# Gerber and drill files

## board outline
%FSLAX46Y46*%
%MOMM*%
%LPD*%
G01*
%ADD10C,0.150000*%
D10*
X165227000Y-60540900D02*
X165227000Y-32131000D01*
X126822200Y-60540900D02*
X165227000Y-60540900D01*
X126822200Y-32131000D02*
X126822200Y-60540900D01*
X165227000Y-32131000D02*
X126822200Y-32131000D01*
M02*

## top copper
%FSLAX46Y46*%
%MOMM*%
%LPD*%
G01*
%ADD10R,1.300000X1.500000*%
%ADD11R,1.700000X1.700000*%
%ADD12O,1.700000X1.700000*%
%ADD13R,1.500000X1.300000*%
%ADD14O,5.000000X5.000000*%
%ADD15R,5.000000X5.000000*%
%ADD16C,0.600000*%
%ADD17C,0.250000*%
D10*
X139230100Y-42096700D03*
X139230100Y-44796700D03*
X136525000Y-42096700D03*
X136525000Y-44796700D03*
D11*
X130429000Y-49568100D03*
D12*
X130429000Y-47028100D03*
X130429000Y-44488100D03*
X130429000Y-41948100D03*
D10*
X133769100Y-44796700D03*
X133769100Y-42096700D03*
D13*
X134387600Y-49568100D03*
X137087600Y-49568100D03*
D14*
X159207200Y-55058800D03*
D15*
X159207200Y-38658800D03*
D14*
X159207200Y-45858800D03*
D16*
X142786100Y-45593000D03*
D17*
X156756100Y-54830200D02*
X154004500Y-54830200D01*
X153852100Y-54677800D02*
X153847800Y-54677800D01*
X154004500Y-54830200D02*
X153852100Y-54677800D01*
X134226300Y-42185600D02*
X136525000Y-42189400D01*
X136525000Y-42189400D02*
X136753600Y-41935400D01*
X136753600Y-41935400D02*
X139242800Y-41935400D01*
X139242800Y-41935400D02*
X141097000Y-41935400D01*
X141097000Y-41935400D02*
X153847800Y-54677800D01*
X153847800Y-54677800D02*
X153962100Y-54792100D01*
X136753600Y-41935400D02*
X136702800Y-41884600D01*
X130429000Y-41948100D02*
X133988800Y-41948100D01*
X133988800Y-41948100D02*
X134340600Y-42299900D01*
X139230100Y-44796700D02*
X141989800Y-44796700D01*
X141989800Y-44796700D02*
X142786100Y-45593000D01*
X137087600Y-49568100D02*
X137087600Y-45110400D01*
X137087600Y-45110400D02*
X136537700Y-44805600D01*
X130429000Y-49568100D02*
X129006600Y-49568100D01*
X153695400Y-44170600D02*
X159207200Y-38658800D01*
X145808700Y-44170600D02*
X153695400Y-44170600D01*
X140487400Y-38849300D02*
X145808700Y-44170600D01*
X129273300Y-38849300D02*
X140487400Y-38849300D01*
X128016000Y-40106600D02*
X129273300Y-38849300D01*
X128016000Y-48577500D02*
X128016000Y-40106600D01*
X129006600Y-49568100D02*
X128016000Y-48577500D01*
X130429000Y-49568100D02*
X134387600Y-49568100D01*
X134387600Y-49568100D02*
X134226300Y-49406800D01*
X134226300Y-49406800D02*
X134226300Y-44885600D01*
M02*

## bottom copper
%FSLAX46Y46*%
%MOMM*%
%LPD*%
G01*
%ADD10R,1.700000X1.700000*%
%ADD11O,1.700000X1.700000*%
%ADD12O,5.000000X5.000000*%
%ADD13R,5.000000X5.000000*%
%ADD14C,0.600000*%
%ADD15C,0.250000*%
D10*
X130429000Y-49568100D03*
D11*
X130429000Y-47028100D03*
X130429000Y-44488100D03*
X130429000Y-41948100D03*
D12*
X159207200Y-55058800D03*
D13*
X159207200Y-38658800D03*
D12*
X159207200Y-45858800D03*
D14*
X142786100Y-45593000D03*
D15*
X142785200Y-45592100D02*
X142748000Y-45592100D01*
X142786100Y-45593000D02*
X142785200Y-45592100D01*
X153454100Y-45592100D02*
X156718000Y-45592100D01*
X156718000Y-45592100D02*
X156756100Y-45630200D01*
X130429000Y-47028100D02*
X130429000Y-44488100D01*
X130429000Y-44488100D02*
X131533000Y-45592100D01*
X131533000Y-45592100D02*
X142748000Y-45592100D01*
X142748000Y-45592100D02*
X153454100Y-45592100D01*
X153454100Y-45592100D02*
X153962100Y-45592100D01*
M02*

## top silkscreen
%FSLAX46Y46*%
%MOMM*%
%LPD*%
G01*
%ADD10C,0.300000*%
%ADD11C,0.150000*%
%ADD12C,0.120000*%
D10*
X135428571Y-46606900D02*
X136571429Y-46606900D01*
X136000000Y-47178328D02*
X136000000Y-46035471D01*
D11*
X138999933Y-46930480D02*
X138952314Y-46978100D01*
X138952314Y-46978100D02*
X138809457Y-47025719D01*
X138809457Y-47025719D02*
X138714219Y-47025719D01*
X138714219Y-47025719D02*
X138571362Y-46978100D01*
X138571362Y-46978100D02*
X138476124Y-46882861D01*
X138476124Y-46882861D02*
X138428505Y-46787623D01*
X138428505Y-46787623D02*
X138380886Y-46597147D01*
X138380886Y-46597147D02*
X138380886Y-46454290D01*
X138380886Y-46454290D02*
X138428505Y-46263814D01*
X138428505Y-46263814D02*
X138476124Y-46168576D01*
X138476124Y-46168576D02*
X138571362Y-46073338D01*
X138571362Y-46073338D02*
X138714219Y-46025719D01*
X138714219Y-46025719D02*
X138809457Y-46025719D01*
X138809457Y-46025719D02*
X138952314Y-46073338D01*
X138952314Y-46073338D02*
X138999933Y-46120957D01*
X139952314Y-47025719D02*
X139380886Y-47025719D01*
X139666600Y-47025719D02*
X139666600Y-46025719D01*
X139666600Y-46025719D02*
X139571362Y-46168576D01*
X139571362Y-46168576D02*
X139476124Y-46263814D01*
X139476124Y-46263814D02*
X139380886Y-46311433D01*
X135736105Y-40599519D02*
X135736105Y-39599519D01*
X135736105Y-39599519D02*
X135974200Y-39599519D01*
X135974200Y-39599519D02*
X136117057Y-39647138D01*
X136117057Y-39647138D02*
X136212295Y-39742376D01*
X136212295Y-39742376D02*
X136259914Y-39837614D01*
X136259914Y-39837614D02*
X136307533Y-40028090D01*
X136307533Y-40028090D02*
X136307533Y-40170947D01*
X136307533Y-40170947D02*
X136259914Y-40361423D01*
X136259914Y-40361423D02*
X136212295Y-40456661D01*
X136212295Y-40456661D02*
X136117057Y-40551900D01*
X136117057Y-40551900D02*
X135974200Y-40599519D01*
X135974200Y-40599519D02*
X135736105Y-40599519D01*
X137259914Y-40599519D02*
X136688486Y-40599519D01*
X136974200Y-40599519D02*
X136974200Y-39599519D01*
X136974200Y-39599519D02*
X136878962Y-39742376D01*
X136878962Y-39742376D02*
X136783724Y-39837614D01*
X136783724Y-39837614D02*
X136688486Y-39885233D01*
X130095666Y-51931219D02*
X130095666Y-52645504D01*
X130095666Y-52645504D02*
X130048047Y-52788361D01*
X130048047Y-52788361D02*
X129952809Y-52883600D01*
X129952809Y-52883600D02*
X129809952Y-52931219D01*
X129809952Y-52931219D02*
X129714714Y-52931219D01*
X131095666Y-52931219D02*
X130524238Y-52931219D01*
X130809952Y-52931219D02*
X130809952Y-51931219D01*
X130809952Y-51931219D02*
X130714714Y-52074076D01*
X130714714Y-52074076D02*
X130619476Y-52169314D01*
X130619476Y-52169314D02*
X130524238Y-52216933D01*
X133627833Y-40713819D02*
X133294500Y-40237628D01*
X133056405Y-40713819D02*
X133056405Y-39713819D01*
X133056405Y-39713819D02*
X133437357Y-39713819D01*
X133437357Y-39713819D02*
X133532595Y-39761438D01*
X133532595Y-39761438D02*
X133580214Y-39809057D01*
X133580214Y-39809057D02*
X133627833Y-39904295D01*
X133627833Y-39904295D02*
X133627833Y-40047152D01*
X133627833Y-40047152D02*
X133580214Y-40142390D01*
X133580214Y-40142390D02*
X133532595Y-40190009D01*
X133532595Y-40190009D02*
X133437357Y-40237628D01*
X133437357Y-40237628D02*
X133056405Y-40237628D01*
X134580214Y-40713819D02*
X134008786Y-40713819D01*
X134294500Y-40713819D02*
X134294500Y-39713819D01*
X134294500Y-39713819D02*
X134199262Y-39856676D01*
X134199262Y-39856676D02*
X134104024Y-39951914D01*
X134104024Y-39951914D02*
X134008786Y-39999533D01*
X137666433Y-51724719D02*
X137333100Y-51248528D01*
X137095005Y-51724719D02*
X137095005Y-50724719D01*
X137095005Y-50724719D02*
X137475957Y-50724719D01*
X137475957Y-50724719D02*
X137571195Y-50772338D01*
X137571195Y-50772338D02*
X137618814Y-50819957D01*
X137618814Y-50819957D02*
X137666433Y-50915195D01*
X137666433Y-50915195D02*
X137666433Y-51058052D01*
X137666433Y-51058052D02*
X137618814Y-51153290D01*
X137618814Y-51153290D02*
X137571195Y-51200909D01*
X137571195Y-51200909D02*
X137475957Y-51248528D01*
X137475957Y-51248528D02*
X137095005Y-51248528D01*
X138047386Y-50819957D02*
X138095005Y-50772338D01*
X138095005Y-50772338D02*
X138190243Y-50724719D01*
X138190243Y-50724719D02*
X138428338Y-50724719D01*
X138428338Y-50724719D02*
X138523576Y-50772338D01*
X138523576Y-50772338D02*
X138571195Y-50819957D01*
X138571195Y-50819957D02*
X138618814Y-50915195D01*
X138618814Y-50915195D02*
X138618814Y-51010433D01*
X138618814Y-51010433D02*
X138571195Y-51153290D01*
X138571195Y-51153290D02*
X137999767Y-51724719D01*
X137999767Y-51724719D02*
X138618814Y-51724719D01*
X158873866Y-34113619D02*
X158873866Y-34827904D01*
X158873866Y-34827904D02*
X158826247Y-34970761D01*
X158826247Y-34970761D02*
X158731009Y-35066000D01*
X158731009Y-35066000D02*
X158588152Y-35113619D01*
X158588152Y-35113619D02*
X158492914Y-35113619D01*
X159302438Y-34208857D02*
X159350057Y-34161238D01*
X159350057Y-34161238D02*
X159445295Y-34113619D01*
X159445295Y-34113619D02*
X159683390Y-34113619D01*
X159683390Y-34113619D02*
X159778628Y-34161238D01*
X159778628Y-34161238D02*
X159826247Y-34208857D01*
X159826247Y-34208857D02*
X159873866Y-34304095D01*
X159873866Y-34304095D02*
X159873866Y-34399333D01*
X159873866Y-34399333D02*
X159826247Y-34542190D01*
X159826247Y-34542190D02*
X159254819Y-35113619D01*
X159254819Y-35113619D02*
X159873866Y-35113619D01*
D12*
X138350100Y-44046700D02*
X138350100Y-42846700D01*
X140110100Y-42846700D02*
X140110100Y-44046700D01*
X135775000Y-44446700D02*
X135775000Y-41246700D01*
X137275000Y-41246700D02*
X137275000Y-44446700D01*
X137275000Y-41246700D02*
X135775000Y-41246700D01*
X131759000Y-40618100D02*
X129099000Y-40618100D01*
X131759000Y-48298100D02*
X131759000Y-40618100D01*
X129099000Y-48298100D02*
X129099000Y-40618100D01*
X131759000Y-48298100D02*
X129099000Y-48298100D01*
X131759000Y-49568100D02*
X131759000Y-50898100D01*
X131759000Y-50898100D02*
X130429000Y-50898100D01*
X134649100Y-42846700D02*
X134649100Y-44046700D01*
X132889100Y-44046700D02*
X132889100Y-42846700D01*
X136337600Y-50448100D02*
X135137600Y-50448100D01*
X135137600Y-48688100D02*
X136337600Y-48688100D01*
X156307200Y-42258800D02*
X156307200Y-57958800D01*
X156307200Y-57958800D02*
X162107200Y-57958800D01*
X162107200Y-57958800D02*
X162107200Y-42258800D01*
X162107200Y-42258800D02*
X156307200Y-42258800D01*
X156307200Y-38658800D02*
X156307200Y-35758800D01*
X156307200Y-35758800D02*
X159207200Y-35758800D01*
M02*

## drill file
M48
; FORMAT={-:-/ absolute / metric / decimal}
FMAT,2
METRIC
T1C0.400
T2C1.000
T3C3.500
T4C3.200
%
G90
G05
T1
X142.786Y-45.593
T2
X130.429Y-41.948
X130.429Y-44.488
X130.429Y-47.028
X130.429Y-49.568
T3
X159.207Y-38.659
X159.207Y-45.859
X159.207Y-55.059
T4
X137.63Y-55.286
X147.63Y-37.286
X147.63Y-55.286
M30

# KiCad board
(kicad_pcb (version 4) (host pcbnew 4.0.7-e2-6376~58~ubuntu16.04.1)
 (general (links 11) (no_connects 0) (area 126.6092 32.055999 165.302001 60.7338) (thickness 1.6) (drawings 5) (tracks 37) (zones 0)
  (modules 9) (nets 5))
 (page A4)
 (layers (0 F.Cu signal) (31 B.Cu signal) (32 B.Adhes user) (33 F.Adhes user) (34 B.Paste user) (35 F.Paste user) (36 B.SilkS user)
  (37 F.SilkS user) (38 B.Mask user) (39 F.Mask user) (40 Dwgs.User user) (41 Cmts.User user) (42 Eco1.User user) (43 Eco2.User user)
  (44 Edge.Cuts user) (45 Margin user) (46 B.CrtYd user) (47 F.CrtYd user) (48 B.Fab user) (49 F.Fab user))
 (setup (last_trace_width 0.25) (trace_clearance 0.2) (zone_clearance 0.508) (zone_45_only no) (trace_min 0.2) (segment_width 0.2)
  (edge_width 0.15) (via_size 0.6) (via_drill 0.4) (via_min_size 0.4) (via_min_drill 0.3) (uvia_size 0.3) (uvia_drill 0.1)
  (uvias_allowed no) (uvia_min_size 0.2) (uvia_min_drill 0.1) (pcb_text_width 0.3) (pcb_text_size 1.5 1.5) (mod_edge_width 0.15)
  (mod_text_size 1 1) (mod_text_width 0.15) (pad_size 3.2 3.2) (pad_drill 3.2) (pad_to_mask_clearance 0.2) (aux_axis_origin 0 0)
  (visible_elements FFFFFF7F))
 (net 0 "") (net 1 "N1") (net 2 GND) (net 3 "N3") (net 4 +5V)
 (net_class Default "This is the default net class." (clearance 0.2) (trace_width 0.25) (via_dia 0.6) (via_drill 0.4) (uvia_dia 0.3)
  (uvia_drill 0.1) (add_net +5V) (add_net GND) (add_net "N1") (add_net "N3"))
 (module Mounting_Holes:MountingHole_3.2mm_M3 (layer F.Cu) (at 137.63 55.286)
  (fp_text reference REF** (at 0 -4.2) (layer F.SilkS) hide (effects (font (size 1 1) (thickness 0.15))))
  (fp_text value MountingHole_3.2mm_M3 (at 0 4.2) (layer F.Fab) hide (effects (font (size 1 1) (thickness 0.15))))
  (pad 1 np_thru_hole circle (at 0 0) (size 3.2 3.2) (drill 3.2) (layers *.Cu *.Mask)))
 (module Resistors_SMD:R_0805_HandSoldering (layer F.Cu) (at 139.2301 43.4467 270)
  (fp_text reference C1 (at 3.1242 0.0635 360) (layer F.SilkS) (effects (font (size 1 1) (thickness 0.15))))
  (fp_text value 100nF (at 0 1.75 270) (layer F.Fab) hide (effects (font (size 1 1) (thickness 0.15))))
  (fp_line (start 0.6 0.88) (end -0.6 0.88) (layer F.SilkS) (width 0.12))
  (fp_line (start -0.6 -0.88) (end 0.6 -0.88) (layer F.SilkS) (width 0.12))
  (pad 1 smd rect (at -1.35 0 270) (size 1.5 1.3) (layers F.Cu F.Paste F.Mask) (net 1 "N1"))
  (pad 2 smd rect (at 1.35 0 270) (size 1.5 1.3) (layers F.Cu F.Paste F.Mask) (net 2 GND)))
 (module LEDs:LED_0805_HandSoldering (layer F.Cu) (at 136.525 43.4467 270)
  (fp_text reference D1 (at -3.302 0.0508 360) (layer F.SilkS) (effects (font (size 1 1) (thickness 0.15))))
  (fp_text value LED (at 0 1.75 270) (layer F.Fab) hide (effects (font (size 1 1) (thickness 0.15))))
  (fp_line (start 1 0.75) (end -2.2 0.75) (layer F.SilkS) (width 0.12))
  (fp_line (start -2.2 -0.75) (end 1 -0.75) (layer F.SilkS) (width 0.12))
  (fp_line (start -2.2 -0.75) (end -2.2 0.75) (layer F.SilkS) (width 0.12))
  (pad 1 smd rect (at -1.35 0 270) (size 1.5 1.3) (layers F.Cu F.Paste F.Mask) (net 1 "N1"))
  (pad 2 smd rect (at 1.35 0 270) (size 1.5 1.3) (layers F.Cu F.Paste F.Mask) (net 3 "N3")))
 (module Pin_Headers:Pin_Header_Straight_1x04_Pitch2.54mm (layer F.Cu) (at 130.429 49.5681 180)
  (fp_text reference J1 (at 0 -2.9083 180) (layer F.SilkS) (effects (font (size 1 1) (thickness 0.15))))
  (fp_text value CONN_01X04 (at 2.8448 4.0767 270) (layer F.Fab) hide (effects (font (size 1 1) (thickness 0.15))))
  (fp_line (start -1.33 8.95) (end 1.33 8.95) (layer F.SilkS) (width 0.12))
  (fp_line (start -1.33 1.27) (end -1.33 8.95) (layer F.SilkS) (width 0.12))
  (fp_line (start 1.33 1.27) (end 1.33 8.95) (layer F.SilkS) (width 0.12))
  (fp_line (start -1.33 1.27) (end 1.33 1.27) (layer F.SilkS) (width 0.12))
  (fp_line (start -1.33 0) (end -1.33 -1.33) (layer F.SilkS) (width 0.12))
  (fp_line (start -1.33 -1.33) (end 0 -1.33) (layer F.SilkS) (width 0.12))
  (pad 1 thru_hole rect (at 0 0 180) (size 1.7 1.7) (drill 1) (layers *.Cu *.Mask) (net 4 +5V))
  (pad 2 thru_hole oval (at 0 2.54 180) (size 1.7 1.7) (drill 1) (layers *.Cu *.Mask) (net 2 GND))
  (pad 3 thru_hole oval (at 0 5.08 180) (size 1.7 1.7) (drill 1) (layers *.Cu *.Mask) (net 2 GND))
  (pad 4 thru_hole oval (at 0 7.62 180) (size 1.7 1.7) (drill 1) (layers *.Cu *.Mask) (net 1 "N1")))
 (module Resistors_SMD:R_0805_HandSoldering (layer F.Cu) (at 133.7691 43.4467 90)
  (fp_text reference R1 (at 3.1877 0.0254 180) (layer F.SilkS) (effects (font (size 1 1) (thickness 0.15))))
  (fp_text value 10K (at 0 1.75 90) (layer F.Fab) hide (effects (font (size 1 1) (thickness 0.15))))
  (fp_line (start 0.6 0.88) (end -0.6 0.88) (layer F.SilkS) (width 0.12))
  (fp_line (start -0.6 -0.88) (end 0.6 -0.88) (layer F.SilkS) (width 0.12))
  (pad 1 smd rect (at -1.35 0 90) (size 1.5 1.3) (layers F.Cu F.Paste F.Mask) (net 4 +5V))
  (pad 2 smd rect (at 1.35 0 90) (size 1.5 1.3) (layers F.Cu F.Paste F.Mask) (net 1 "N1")))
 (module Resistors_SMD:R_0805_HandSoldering (layer F.Cu) (at 135.7376 49.5681)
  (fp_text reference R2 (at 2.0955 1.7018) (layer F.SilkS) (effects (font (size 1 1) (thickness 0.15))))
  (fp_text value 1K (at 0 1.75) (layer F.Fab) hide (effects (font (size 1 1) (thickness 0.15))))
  (fp_line (start 0.6 0.88) (end -0.6 0.88) (layer F.SilkS) (width 0.12))
  (fp_line (start -0.6 -0.88) (end 0.6 -0.88) (layer F.SilkS) (width 0.12))
  (pad 1 smd rect (at -1.35 0) (size 1.5 1.3) (layers F.Cu F.Paste F.Mask) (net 4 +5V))
  (pad 2 smd rect (at 1.35 0) (size 1.5 1.3) (layers F.Cu F.Paste F.Mask) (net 3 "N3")))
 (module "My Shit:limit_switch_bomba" (layer F.Cu) (at 159.2072 38.6588)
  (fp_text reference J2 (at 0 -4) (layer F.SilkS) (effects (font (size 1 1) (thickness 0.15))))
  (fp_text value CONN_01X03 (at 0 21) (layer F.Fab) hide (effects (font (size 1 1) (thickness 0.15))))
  (fp_line (start -2.9 3.6) (end -2.9 19.3) (layer F.SilkS) (width 0.12))
  (fp_line (start -2.9 19.3) (end 2.9 19.3) (layer F.SilkS) (width 0.12))
  (fp_line (start 2.9 19.3) (end 2.9 3.6) (layer F.SilkS) (width 0.12))
  (fp_line (start 2.9 3.6) (end -2.9 3.6) (layer F.SilkS) (width 0.12))
  (fp_line (start -2.9 0) (end -2.9 -2.9) (layer F.SilkS) (width 0.12))
  (fp_line (start -2.9 -2.9) (end 0 -2.9) (layer F.SilkS) (width 0.12))
  (pad 1 thru_hole oval (at 0 16.4) (size 5 5) (drill 3.5) (layers *.Cu *.Mask) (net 1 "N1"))
  (pad 2 thru_hole rect (at 0 0) (size 5 5) (drill 3.5) (layers *.Cu *.Mask) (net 4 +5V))
  (pad 3 thru_hole oval (at 0 7.2) (size 5 5) (drill 3.5) (layers *.Cu *.Mask) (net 2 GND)))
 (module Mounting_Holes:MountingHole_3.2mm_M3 (layer F.Cu) (at 147.63 37.286)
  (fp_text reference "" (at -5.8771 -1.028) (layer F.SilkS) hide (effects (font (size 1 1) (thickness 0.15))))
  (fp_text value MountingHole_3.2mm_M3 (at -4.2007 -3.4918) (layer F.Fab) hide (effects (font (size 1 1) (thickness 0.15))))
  (pad 1 np_thru_hole circle (at 0 0) (size 3.2 3.2) (drill 3.2) (layers *.Cu *.Mask)))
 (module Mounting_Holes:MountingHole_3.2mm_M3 (layer F.Cu) (at 147.63 55.286)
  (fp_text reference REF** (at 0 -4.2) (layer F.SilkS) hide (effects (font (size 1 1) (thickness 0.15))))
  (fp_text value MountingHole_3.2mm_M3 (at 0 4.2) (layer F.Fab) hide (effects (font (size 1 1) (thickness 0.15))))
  (pad 1 np_thru_hole circle (at 0 0) (size 3.2 3.2) (drill 3.2) (layers *.Cu *.Mask)))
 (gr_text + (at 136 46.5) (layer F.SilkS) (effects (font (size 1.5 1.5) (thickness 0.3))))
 (gr_line (start 165.227 60.5409) (end 165.227 32.131) (angle 90) (layer Edge.Cuts) (width 0.15))
 (gr_line (start 126.8222 60.5409) (end 165.227 60.5409) (angle 90) (layer Edge.Cuts) (width 0.15))
 (gr_line (start 126.8222 32.131) (end 126.8222 60.5409) (angle 90) (layer Edge.Cuts) (width 0.15))
 (gr_line (start 165.227 32.131) (end 126.8222 32.131) (angle 90) (layer Edge.Cuts) (width 0.15))
 (segment (start 156.7561 54.8302) (end 154.0045 54.8302) (width 0.25) (layer F.Cu) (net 1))
 (segment (start 153.8521 54.6778) (end 153.8478 54.6778) (width 0.25) (layer F.Cu) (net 1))
 (segment (start 154.0045 54.8302) (end 153.8521 54.6778) (width 0.25) (layer F.Cu) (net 1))
 (segment (start 134.2263 42.1856) (end 136.525 42.1894) (width 0.25) (layer F.Cu) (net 1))
 (segment (start 136.525 42.1894) (end 136.7536 41.9354) (width 0.25) (layer F.Cu) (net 1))
 (segment (start 136.7536 41.9354) (end 139.2428 41.9354) (width 0.25) (layer F.Cu) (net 1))
 (segment (start 139.2428 41.9354) (end 141.097 41.9354) (width 0.25) (layer F.Cu) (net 1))
 (segment (start 141.097 41.9354) (end 153.8478 54.6778) (width 0.25) (layer F.Cu) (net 1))
 (segment (start 153.8478 54.6778) (end 153.9621 54.7921) (width 0.25) (layer F.Cu) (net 1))
 (segment (start 136.7536 41.9354) (end 136.7028 41.8846) (width 0.25) (layer F.Cu) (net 1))
 (segment (start 130.429 41.9481) (end 133.9888 41.9481) (width 0.25) (layer F.Cu) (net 1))
 (segment (start 133.9888 41.9481) (end 134.3406 42.2999) (width 0.25) (layer F.Cu) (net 1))
 (segment (start 139.2301 44.7967) (end 141.9898 44.7967) (width 0.25) (layer F.Cu) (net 2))
 (segment (start 142.7852 45.5921) (end 142.748 45.5921) (width 0.25) (layer B.Cu) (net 2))
 (segment (start 142.7861 45.593) (end 142.7852 45.5921) (width 0.25) (layer B.Cu) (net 2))
 (via (at 142.7861 45.593) (size 0.6) (drill 0.4) (layers F.Cu B.Cu) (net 2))
 (segment (start 141.9898 44.7967) (end 142.7861 45.593) (width 0.25) (layer F.Cu) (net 2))
 (segment (start 153.4541 45.5921) (end 156.718 45.5921) (width 0.25) (layer B.Cu) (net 2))
 (segment (start 156.718 45.5921) (end 156.7561 45.6302) (width 0.25) (layer B.Cu) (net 2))
 (segment (start 130.429 47.0281) (end 130.429 44.4881) (width 0.25) (layer B.Cu) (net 2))
 (segment (start 130.429 44.4881) (end 131.533 45.5921) (width 0.25) (layer B.Cu) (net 2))
 (segment (start 131.533 45.5921) (end 142.748 45.5921) (width 0.25) (layer B.Cu) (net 2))
 (segment (start 142.748 45.5921) (end 153.4541 45.5921) (width 0.25) (layer B.Cu) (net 2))
 (segment (start 153.4541 45.5921) (end 153.9621 45.5921) (width 0.25) (layer B.Cu) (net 2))
 (segment (start 137.0876 49.5681) (end 137.0876 45.1104) (width 0.25) (layer F.Cu) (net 3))
 (segment (start 137.0876 45.1104) (end 136.5377 44.8056) (width 0.25) (layer F.Cu) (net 3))
 (segment (start 130.429 49.5681) (end 129.0066 49.5681) (width 0.25) (layer F.Cu) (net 4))
 (segment (start 153.6954 44.1706) (end 159.2072 38.6588) (width 0.25) (layer F.Cu) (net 4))
 (segment (start 145.8087 44.1706) (end 153.6954 44.1706) (width 0.25) (layer F.Cu) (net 4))
 (segment (start 140.4874 38.8493) (end 145.8087 44.1706) (width 0.25) (layer F.Cu) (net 4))
 (segment (start 129.2733 38.8493) (end 140.4874 38.8493) (width 0.25) (layer F.Cu) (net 4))
 (segment (start 128.016 40.1066) (end 129.2733 38.8493) (width 0.25) (layer F.Cu) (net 4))
 (segment (start 128.016 48.5775) (end 128.016 40.1066) (width 0.25) (layer F.Cu) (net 4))
 (segment (start 129.0066 49.5681) (end 128.016 48.5775) (width 0.25) (layer F.Cu) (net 4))
 (segment (start 130.429 49.5681) (end 134.3876 49.5681) (width 0.25) (layer F.Cu) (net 4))
 (segment (start 134.3876 49.5681) (end 134.2263 49.4068) (width 0.25) (layer F.Cu) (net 4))
 (segment (start 134.2263 49.4068) (end 134.2263 44.8856) (width 0.25) (layer F.Cu) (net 4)))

